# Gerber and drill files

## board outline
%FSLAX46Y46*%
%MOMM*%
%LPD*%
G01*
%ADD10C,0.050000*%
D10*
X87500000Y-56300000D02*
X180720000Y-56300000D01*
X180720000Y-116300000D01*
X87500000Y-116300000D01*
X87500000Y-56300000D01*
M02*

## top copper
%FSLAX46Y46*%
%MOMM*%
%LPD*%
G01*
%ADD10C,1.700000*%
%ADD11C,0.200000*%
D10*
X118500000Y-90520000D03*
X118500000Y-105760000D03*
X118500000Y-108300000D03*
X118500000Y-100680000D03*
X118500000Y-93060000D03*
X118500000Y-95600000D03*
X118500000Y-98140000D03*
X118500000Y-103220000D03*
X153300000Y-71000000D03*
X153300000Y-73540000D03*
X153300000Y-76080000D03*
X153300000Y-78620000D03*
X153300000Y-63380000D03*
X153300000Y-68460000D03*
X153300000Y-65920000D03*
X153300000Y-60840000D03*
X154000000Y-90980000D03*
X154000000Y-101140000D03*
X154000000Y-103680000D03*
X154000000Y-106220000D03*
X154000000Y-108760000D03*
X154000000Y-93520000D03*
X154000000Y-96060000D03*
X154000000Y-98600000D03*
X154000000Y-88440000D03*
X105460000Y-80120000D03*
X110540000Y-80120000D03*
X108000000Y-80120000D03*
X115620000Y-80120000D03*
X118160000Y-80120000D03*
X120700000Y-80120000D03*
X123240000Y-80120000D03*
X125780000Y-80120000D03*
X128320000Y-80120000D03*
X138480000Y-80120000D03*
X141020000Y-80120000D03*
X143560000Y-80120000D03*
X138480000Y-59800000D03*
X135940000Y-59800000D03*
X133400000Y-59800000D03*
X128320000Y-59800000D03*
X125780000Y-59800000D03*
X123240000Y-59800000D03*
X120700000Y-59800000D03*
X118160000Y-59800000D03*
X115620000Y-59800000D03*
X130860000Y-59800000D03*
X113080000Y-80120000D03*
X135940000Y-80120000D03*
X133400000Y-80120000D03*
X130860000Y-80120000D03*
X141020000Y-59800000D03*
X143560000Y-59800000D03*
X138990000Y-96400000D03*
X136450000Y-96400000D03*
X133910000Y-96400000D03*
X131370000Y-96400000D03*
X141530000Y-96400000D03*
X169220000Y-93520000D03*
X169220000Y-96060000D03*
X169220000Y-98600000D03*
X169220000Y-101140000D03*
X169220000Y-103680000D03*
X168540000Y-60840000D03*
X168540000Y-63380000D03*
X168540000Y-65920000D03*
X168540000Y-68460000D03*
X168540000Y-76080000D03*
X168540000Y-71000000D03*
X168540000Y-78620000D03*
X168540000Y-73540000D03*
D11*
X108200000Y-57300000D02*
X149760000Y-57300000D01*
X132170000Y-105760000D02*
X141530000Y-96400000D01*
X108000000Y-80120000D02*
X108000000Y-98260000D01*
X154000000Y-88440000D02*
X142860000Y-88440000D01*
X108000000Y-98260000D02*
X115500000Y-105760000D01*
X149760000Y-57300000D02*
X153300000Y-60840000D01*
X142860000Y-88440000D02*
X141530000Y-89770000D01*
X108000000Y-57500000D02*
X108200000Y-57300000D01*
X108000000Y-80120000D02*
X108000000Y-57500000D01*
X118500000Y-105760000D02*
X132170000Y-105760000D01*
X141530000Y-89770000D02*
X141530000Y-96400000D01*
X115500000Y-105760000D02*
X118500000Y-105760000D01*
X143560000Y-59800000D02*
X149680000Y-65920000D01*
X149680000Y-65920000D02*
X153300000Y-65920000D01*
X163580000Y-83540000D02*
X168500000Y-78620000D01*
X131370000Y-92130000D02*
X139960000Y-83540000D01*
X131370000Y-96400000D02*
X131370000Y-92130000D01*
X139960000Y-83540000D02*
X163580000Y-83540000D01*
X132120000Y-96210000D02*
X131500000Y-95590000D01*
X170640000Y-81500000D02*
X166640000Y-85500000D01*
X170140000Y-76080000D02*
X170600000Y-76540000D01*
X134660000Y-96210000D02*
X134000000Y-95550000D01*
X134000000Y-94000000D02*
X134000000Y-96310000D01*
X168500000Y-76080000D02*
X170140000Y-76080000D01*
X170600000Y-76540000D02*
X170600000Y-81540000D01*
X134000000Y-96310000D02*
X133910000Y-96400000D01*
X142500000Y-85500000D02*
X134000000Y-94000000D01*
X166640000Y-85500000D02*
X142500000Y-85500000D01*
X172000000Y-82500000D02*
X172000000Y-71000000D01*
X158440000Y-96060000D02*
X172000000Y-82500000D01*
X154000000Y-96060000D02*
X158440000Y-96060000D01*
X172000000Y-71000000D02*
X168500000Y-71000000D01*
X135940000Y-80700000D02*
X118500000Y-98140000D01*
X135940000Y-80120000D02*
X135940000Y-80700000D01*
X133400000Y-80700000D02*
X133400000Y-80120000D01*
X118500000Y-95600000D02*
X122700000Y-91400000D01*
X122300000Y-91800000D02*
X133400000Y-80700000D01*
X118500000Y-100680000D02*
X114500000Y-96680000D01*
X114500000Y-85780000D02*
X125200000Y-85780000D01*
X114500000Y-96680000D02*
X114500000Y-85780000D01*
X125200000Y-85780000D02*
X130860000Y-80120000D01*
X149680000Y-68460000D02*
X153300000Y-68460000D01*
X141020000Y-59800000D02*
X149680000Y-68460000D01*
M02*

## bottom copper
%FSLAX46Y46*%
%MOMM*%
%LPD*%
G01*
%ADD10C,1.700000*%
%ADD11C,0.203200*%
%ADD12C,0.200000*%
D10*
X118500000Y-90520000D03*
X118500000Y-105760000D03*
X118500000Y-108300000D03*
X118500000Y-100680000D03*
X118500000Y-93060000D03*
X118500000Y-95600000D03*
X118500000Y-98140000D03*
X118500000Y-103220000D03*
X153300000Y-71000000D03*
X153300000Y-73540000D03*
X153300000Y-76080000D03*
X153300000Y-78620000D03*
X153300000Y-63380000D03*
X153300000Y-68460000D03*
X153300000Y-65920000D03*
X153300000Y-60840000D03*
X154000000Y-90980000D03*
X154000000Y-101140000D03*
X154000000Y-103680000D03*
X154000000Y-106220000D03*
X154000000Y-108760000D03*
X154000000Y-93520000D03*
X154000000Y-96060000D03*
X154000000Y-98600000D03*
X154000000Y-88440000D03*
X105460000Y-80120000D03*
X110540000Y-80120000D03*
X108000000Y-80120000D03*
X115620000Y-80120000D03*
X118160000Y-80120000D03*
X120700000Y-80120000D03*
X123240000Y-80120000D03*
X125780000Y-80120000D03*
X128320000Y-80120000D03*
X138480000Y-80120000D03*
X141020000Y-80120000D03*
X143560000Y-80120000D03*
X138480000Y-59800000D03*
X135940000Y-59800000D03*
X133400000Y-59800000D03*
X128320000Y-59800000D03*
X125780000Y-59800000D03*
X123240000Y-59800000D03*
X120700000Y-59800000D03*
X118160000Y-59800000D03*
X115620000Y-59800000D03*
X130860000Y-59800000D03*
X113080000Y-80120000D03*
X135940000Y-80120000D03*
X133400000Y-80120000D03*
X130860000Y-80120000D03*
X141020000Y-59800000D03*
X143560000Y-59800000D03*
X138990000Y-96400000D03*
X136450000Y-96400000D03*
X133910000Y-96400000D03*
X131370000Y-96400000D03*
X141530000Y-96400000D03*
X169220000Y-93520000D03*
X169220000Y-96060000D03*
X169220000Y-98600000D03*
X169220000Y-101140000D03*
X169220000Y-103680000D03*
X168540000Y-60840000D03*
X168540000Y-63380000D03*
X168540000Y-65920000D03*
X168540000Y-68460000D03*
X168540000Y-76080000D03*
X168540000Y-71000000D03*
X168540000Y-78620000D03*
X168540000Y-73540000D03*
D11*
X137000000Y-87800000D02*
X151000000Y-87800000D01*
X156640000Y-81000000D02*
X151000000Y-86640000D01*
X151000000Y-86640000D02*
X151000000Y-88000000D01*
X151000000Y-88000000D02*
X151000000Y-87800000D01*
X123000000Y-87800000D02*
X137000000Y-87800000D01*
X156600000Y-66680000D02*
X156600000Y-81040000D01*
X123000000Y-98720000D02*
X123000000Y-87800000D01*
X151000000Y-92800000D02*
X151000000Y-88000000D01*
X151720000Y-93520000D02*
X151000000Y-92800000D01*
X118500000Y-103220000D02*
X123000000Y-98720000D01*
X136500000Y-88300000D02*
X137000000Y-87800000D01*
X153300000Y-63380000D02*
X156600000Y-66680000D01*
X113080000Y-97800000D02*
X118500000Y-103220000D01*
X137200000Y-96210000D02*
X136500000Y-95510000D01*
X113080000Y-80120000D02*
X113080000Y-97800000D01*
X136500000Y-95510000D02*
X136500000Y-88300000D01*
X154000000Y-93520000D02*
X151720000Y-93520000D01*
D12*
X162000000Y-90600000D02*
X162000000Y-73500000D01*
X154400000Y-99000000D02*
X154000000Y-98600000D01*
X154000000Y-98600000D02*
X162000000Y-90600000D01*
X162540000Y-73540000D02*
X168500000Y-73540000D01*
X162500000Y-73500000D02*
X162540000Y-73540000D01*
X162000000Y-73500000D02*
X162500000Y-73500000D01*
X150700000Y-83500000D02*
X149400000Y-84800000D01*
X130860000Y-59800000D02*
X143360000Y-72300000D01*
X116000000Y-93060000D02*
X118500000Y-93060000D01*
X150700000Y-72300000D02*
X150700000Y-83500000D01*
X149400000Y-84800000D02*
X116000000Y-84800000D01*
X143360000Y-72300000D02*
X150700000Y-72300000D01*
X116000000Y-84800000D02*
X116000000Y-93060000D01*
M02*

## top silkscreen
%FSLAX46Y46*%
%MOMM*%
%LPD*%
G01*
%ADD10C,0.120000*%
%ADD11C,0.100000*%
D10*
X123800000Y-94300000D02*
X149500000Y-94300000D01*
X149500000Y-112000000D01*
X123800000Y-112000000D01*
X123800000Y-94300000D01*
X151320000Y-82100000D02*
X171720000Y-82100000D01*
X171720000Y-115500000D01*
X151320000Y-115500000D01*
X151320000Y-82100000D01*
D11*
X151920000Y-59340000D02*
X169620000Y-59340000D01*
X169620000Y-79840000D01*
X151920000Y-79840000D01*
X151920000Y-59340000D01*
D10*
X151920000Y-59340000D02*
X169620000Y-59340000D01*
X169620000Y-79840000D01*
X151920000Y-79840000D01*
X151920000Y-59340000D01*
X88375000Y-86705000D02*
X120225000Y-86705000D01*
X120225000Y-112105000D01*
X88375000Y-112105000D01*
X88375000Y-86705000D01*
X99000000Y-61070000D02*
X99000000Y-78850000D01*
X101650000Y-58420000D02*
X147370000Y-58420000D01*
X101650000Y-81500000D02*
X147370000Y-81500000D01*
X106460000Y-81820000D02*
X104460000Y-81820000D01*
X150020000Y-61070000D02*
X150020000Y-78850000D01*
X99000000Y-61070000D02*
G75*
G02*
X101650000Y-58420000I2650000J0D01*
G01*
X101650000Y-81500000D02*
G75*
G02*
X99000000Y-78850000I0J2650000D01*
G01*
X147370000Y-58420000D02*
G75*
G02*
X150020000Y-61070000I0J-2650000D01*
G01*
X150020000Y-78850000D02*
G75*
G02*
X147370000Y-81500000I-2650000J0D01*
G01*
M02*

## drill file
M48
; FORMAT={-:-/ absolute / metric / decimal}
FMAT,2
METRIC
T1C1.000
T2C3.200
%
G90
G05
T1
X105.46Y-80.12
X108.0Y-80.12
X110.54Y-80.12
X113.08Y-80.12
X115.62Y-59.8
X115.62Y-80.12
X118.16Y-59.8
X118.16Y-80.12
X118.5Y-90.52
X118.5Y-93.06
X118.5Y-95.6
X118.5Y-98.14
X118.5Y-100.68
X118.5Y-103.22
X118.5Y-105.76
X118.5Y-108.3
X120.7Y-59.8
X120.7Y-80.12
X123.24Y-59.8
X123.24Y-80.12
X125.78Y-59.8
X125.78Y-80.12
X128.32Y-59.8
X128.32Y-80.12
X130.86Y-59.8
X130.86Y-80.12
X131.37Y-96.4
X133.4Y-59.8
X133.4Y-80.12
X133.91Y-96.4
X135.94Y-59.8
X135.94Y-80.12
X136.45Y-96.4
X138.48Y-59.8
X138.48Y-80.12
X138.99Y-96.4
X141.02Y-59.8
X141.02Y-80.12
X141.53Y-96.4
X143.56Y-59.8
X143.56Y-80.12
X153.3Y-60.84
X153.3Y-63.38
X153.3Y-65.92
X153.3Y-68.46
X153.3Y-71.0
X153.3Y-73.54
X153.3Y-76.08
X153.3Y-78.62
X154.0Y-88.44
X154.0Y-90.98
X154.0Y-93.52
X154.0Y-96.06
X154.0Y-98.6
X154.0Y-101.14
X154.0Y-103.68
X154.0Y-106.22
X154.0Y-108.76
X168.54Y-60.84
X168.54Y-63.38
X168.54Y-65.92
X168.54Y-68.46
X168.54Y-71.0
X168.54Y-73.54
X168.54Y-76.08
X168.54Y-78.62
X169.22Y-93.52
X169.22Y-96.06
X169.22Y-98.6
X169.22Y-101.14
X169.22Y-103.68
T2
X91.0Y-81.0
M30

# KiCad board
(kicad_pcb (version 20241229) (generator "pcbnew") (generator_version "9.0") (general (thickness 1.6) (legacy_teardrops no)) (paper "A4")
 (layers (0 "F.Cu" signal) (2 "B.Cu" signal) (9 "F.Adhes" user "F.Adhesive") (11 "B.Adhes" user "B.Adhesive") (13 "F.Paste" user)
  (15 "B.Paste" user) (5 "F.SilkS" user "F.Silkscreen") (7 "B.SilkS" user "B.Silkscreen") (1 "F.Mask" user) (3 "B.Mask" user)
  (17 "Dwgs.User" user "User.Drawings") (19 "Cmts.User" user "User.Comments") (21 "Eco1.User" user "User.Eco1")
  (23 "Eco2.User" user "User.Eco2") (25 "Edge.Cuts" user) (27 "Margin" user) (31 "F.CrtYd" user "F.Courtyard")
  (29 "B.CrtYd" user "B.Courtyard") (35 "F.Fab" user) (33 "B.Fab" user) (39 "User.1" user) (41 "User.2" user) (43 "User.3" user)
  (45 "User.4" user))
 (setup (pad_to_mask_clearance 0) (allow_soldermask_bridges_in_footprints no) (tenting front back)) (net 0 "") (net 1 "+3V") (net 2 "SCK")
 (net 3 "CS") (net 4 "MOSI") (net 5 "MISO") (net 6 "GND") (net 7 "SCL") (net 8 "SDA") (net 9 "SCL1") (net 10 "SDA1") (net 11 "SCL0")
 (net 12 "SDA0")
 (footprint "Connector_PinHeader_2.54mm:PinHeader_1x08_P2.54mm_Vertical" (layer "F.Cu") (at 118.5 90.52)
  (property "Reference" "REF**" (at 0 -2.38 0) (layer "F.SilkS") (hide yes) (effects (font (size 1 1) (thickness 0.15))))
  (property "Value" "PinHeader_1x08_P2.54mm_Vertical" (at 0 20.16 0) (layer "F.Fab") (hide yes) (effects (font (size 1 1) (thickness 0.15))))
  (pad "1" thru_hole circle (at 0 0) (size 1.7 1.7) (drill 1) (layers "*.Cu" "*.Mask") (remove_unused_layers no))
  (pad "3V" thru_hole circle (at 0 15.24) (size 1.7 1.7) (drill 1) (layers "*.Cu" "*.Mask") (remove_unused_layers no) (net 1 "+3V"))
  (pad "8" thru_hole circle (at 0 17.78) (size 1.7 1.7) (drill 1) (layers "*.Cu" "*.Mask") (remove_unused_layers no))
  (pad "CLK" thru_hole circle (at 0 10.16) (size 1.7 1.7) (drill 1) (layers "*.Cu" "*.Mask") (remove_unused_layers no) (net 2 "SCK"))
  (pad "CS" thru_hole circle (at 0 2.54) (size 1.7 1.7) (drill 1) (layers "*.Cu" "*.Mask") (remove_unused_layers no) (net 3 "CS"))
  (pad "DI" thru_hole circle (at 0 5.08) (size 1.7 1.7) (drill 1) (layers "*.Cu" "*.Mask") (remove_unused_layers no) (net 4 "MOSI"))
  (pad "DO" thru_hole circle (at 0 7.62) (size 1.7 1.7) (drill 1) (layers "*.Cu" "*.Mask") (remove_unused_layers no) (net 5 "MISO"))
  (pad "GND" thru_hole circle (at 0 12.7) (size 1.7 1.7) (drill 1) (layers "*.Cu" "*.Mask") (remove_unused_layers no) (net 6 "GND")))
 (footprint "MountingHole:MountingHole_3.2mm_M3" (layer "F.Cu") (at 91 81)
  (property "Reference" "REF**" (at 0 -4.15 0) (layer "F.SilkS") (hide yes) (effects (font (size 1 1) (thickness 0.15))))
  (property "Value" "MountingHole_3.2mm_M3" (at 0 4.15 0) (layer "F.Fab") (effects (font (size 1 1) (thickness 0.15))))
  (pad "" np_thru_hole circle (at 0 0) (size 3.2 3.2) (drill 3.2) (layers "*.Cu" "*.Mask")))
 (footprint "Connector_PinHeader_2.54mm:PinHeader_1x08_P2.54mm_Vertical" (layer "F.Cu") (at 153.3 60.84)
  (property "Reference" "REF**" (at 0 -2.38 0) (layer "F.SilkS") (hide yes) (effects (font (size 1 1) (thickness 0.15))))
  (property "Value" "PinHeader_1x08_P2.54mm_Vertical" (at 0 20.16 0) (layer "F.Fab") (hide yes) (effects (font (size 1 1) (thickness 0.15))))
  (pad "5" thru_hole circle (at 0 10.16) (size 1.7 1.7) (drill 1) (layers "*.Cu" "*.Mask") (remove_unused_layers no))
  (pad "6" thru_hole circle (at 0 12.7) (size 1.7 1.7) (drill 1) (layers "*.Cu" "*.Mask") (remove_unused_layers no))
  (pad "7" thru_hole circle (at 0 15.24) (size 1.7 1.7) (drill 1) (layers "*.Cu" "*.Mask") (remove_unused_layers no))
  (pad "8" thru_hole circle (at 0 17.78) (size 1.7 1.7) (drill 1) (layers "*.Cu" "*.Mask") (remove_unused_layers no))
  (pad "GND" thru_hole circle (at 0 2.54) (size 1.7 1.7) (drill 1) (layers "*.Cu" "*.Mask") (remove_unused_layers no) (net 6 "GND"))
  (pad "SCL" thru_hole circle (at 0 7.62) (size 1.7 1.7) (drill 1) (layers "*.Cu" "*.Mask") (remove_unused_layers no) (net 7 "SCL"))
  (pad "SDA" thru_hole circle (at 0 5.08) (size 1.7 1.7) (drill 1) (layers "*.Cu" "*.Mask") (remove_unused_layers no) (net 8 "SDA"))
  (pad "VIN" thru_hole circle (at 0 0) (size 1.7 1.7) (drill 1) (layers "*.Cu" "*.Mask") (remove_unused_layers no) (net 1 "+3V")))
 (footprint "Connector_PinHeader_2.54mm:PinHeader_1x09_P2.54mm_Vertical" (layer "F.Cu") (at 154 88.44)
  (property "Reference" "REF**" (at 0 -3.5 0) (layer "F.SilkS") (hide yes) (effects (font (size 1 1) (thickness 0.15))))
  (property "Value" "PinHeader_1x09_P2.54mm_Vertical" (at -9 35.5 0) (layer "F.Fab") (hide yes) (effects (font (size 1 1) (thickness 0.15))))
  (pad "2" thru_hole circle (at 0 2.54) (size 1.7 1.7) (drill 1) (layers "*.Cu" "*.Mask") (remove_unused_layers no))
  (pad "6" thru_hole circle (at 0 12.7) (size 1.7 1.7) (drill 1) (layers "*.Cu" "*.Mask") (remove_unused_layers no))
  (pad "7" thru_hole circle (at 0 15.24) (size 1.7 1.7) (drill 1) (layers "*.Cu" "*.Mask") (remove_unused_layers no))
  (pad "8" thru_hole circle (at 0 17.78) (size 1.7 1.7) (drill 1) (layers "*.Cu" "*.Mask") (remove_unused_layers no))
  (pad "9" thru_hole circle (at 0 20.32) (size 1.7 1.7) (drill 1) (layers "*.Cu" "*.Mask") (remove_unused_layers no))
  (pad "GND" thru_hole circle (at 0 5.08) (size 1.7 1.7) (drill 1) (layers "*.Cu" "*.Mask") (remove_unused_layers no) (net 6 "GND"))
  (pad "SCL" thru_hole circle (at 0 7.62) (size 1.7 1.7) (drill 1) (layers "*.Cu" "*.Mask") (remove_unused_layers no) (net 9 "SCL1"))
  (pad "SDA" thru_hole circle (at 0 10.16) (size 1.7 1.7) (drill 1) (layers "*.Cu" "*.Mask") (remove_unused_layers no) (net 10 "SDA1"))
  (pad "VIN" thru_hole circle (at 0 0) (size 1.7 1.7) (drill 1) (layers "*.Cu" "*.Mask") (remove_unused_layers no) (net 1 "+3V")))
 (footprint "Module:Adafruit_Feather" (layer "F.Cu") (at 105.46 80.12 90)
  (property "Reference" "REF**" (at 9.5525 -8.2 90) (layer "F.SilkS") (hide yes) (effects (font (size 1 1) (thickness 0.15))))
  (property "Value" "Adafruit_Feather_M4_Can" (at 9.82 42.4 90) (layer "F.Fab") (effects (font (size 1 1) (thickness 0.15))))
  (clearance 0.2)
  (fp_line (start 19.05 -6.46) (end 1.27 -6.46) (stroke (width 0.12) (type solid)) (layer "F.SilkS"))
  (fp_line (start 21.7 -3.81) (end 21.7 41.91) (stroke (width 0.12) (type solid)) (layer "F.SilkS"))
  (fp_line (start -1.38 -3.81) (end -1.38 41.91) (stroke (width 0.12) (type solid)) (layer "F.SilkS"))
  (fp_line (start -1.7 1) (end -1.7 -1) (stroke (width 0.12) (type solid)) (layer "F.SilkS"))
  (fp_line (start 19.05 44.56) (end 1.27 44.56) (stroke (width 0.12) (type solid)) (layer "F.SilkS"))
  (fp_arc (start 19.05 -6.46) (mid 20.923833 -5.683833) (end 21.7 -3.81) (stroke (width 0.12) (type solid)) (layer "F.SilkS"))
  (fp_arc (start -1.38 -3.81) (mid -0.603833 -5.683833) (end 1.27 -6.46) (stroke (width 0.12) (type solid)) (layer "F.SilkS"))
  (fp_arc (start 21.7 41.91) (mid 20.923833 43.783833) (end 19.05 44.56) (stroke (width 0.12) (type solid)) (layer "F.SilkS"))
  (fp_arc (start 1.27 44.56) (mid -0.603833 43.783833) (end -1.38 41.91) (stroke (width 0.12) (type solid)) (layer "F.SilkS"))
  (pad "1" thru_hole circle (at 0 0 90) (size 1.7 1.7) (drill 1) (layers "*.Cu" "*.Mask") (remove_unused_layers no))
  (pad "3" thru_hole circle (at 0 5.08 90) (size 1.7 1.7) (drill 1) (layers "*.Cu" "*.Mask") (remove_unused_layers no))
  (pad "3V" thru_hole circle (at 0 2.54 90) (size 1.7 1.7) (drill 1) (layers "*.Cu" "*.Mask") (remove_unused_layers no) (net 1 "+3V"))
  (pad "5" thru_hole circle (at 0 10.16 90) (size 1.7 1.7) (drill 1) (layers "*.Cu" "*.Mask") (remove_unused_layers no))
  (pad "6" thru_hole circle (at 0 12.7 90) (size 1.7 1.7) (drill 1) (layers "*.Cu" "*.Mask") (remove_unused_layers no))
  (pad "7" thru_hole circle (at 0 15.24 90) (size 1.7 1.7) (drill 1) (layers "*.Cu" "*.Mask") (remove_unused_layers no))
  (pad "8" thru_hole circle (at 0 17.78 90) (size 1.7 1.7) (drill 1) (layers "*.Cu" "*.Mask") (remove_unused_layers no))
  (pad "9" thru_hole circle (at 0 20.32 90) (size 1.7 1.7) (drill 1) (layers "*.Cu" "*.Mask") (remove_unused_layers no))
  (pad "10" thru_hole circle (at 0 22.86 90) (size 1.7 1.7) (drill 1) (layers "*.Cu" "*.Mask") (remove_unused_layers no))
  (pad "14" thru_hole circle (at 0 33.02 90) (size 1.7 1.7) (drill 1) (layers "*.Cu" "*.Mask") (remove_unused_layers no))
  (pad "15" thru_hole circle (at 0 35.56 90) (size 1.7 1.7) (drill 1) (layers "*.Cu" "*.Mask") (remove_unused_layers no))
  (pad "16" thru_hole circle (at 0 38.1 90) (size 1.7 1.7) (drill 1) (layers "*.Cu" "*.Mask") (remove_unused_layers no))
  (pad "19" thru_hole circle (at 20.32 33.02 270) (size 1.7 1.7) (drill 1) (layers "*.Cu" "*.Mask") (remove_unused_layers no))
  (pad "20" thru_hole circle (at 20.32 30.48 270) (size 1.7 1.7) (drill 1) (layers "*.Cu" "*.Mask") (remove_unused_layers no))
  (pad "21" thru_hole circle (at 20.32 27.94 270) (size 1.7 1.7) (drill 1) (layers "*.Cu" "*.Mask") (remove_unused_layers no))
  (pad "23" thru_hole circle (at 20.32 22.86 270) (size 1.7 1.7) (drill 1) (layers "*.Cu" "*.Mask") (remove_unused_layers no))
  (pad "24" thru_hole circle (at 20.32 20.32 270) (size 1.7 1.7) (drill 1) (layers "*.Cu" "*.Mask") (remove_unused_layers no))
  (pad "25" thru_hole circle (at 20.32 17.78 270) (size 1.7 1.7) (drill 1) (layers "*.Cu" "*.Mask") (remove_unused_layers no))
  (pad "26" thru_hole circle (at 20.32 15.24 270) (size 1.7 1.7) (drill 1) (layers "*.Cu" "*.Mask") (remove_unused_layers no))
  (pad "27" thru_hole circle (at 20.32 12.7 270) (size 1.7 1.7) (drill 1) (layers "*.Cu" "*.Mask") (remove_unused_layers no))
  (pad "28" thru_hole circle (at 20.32 10.16 270) (size 1.7 1.7) (drill 1) (layers "*.Cu" "*.Mask") (remove_unused_layers no))
  (pad "D10" thru_hole circle (at 20.32 25.4 270) (size 1.7 1.7) (drill 1) (layers "*.Cu" "*.Mask") (remove_unused_layers no) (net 3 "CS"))
  (pad "GND" thru_hole circle (at 0 7.62 90) (size 1.7 1.7) (drill 1) (layers "*.Cu" "*.Mask") (remove_unused_layers no) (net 6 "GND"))
  (pad "MIS" thru_hole circle (at 0 30.48 90) (size 1.7 1.7) (drill 1) (layers "*.Cu" "*.Mask") (remove_unused_layers no) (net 5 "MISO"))
  (pad "MOSI" thru_hole circle (at 0 27.94 90) (size 1.7 1.7) (drill 1) (layers "*.Cu" "*.Mask") (remove_unused_layers no) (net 4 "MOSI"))
  (pad "SCK" thru_hole circle (at 0 25.4 90) (size 1.7 1.7) (drill 1) (layers "*.Cu" "*.Mask") (remove_unused_layers no) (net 2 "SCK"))
  (pad "SCL" thru_hole circle (at 20.32 35.56 270) (size 1.7 1.7) (drill 1) (layers "*.Cu" "*.Mask") (remove_unused_layers no) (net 7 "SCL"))
  (pad "SDA" thru_hole circle (at 20.32 38.1 270) (size 1.7 1.7) (drill 1) (layers "*.Cu" "*.Mask") (remove_unused_layers no) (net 8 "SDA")))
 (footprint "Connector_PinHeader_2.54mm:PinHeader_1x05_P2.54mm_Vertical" (layer "F.Cu") (at 131.37 96.4 90)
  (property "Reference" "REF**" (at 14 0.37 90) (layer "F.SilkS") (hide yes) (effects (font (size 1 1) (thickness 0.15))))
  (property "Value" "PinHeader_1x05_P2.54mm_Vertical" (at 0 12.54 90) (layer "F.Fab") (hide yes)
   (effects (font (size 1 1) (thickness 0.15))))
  (pad "4" thru_hole circle (at 0 7.62 90) (size 1.7 1.7) (drill 1) (layers "*.Cu" "*.Mask") (remove_unused_layers no))
  (pad "GND" thru_hole circle (at 0 5.08 90) (size 1.7 1.7) (drill 1) (layers "*.Cu" "*.Mask") (remove_unused_layers no) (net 6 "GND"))
  (pad "SCL" thru_hole circle (at 0 2.54 90) (size 1.7 1.7) (drill 1) (layers "*.Cu" "*.Mask") (remove_unused_layers no) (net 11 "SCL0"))
  (pad "SDA" thru_hole circle (at 0 0 90) (size 1.7 1.7) (drill 1) (layers "*.Cu" "*.Mask") (remove_unused_layers no) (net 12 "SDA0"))
  (pad "VIN" thru_hole circle (at 0 10.16 90) (size 1.7 1.7) (drill 1) (layers "*.Cu" "*.Mask") (remove_unused_layers no) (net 1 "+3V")))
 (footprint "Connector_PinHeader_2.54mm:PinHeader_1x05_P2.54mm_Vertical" (layer "F.Cu") (at 169.22 93.52)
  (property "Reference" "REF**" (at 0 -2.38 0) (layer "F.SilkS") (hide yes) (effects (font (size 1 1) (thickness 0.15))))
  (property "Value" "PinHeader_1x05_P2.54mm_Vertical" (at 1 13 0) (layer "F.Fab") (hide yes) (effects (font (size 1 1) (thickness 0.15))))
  (pad "1" thru_hole circle (at 0 0) (size 1.7 1.7) (drill 1) (layers "*.Cu" "*.Mask") (remove_unused_layers no))
  (pad "2" thru_hole circle (at 0 2.54) (size 1.7 1.7) (drill 1) (layers "*.Cu" "*.Mask") (remove_unused_layers no))
  (pad "3" thru_hole circle (at 0 5.08) (size 1.7 1.7) (drill 1) (layers "*.Cu" "*.Mask") (remove_unused_layers no))
  (pad "4" thru_hole circle (at 0 7.62) (size 1.7 1.7) (drill 1) (layers "*.Cu" "*.Mask") (remove_unused_layers no))
  (pad "5" thru_hole circle (at 0 10.16) (size 1.7 1.7) (drill 1) (layers "*.Cu" "*.Mask") (remove_unused_layers no)))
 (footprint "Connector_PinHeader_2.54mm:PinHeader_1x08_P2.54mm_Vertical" (layer "F.Cu") (at 168.54 60.84)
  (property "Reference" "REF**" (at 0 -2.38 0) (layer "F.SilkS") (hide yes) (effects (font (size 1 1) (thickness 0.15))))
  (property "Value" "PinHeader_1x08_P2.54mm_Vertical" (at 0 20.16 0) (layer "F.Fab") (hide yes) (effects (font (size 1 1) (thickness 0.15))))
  (pad "1" thru_hole circle (at 0 0) (size 1.7 1.7) (drill 1) (layers "*.Cu" "*.Mask") (remove_unused_layers no))
  (pad "2" thru_hole circle (at 0 2.54) (size 1.7 1.7) (drill 1) (layers "*.Cu" "*.Mask") (remove_unused_layers no))
  (pad "3" thru_hole circle (at 0 5.08) (size 1.7 1.7) (drill 1) (layers "*.Cu" "*.Mask") (remove_unused_layers no))
  (pad "4" thru_hole circle (at 0 7.62) (size 1.7 1.7) (drill 1) (layers "*.Cu" "*.Mask") (remove_unused_layers no))
  (pad "SC0" thru_hole circle (at 0 15.24) (size 1.7 1.7) (drill 1) (layers "*.Cu" "*.Mask") (remove_unused_layers no) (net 11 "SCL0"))
  (pad "SC1" thru_hole circle (at 0 10.16) (size 1.7 1.7) (drill 1) (layers "*.Cu" "*.Mask") (remove_unused_layers no) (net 9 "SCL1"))
  (pad "SD0" thru_hole circle (at 0 17.78) (size 1.7 1.7) (drill 1) (layers "*.Cu" "*.Mask") (remove_unused_layers no) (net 12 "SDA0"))
  (pad "SD1" thru_hole circle (at 0 12.7) (size 1.7 1.7) (drill 1) (layers "*.Cu" "*.Mask") (remove_unused_layers no) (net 10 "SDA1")))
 (gr_rect (start 123.8 94.3) (end 149.5 112) (stroke (width 0.12) (type solid)) (fill no) (layer "F.SilkS"))
 (gr_rect (start 151.32 82.1) (end 171.72 115.5) (stroke (width 0.12) (type solid)) (fill no) (layer "F.SilkS"))
 (gr_rect (start 151.92 59.34) (end 169.62 79.84) (stroke (width 0.1) (type solid)) (fill no) (layer "F.SilkS"))
 (gr_rect (start 151.92 59.34) (end 169.62 79.84) (stroke (width 0.12) (type solid)) (fill no) (layer "F.SilkS"))
 (gr_rect (start 88.375 86.705) (end 120.225 112.105) (stroke (width 0.12) (type solid)) (fill no) (layer "F.SilkS"))
 (gr_rect (start 87.5 56.3) (end 180.72 116.3) (stroke (width 0.05) (type solid)) (fill no) (layer "Edge.Cuts"))
 (segment (start 108.2 57.3) (end 149.76 57.3) (width 0.2) (layer "F.Cu") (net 1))
 (segment (start 132.17 105.76) (end 141.53 96.4) (width 0.2) (layer "F.Cu") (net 1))
 (segment (start 108 80.12) (end 108 98.26) (width 0.2) (layer "F.Cu") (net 1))
 (segment (start 154 88.44) (end 142.86 88.44) (width 0.2) (layer "F.Cu") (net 1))
 (segment (start 108 98.26) (end 115.5 105.76) (width 0.2) (layer "F.Cu") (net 1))
 (segment (start 149.76 57.3) (end 153.3 60.84) (width 0.2) (layer "F.Cu") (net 1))
 (segment (start 142.86 88.44) (end 141.53 89.77) (width 0.2) (layer "F.Cu") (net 1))
 (segment (start 108 57.5) (end 108.2 57.3) (width 0.2) (layer "F.Cu") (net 1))
 (segment (start 108 80.12) (end 108 57.5) (width 0.2) (layer "F.Cu") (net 1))
 (segment (start 118.5 105.76) (end 132.17 105.76) (width 0.2) (layer "F.Cu") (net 1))
 (segment (start 141.53 89.77) (end 141.53 96.4) (width 0.2) (layer "F.Cu") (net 1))
 (segment (start 115.5 105.76) (end 118.5 105.76) (width 0.2) (layer "F.Cu") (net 1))
 (segment (start 137 87.8) (end 151 87.8) (width 0.2032) (layer "B.Cu") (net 6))
 (segment (start 156.64 81) (end 151 86.64) (width 0.2032) (layer "B.Cu") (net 6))
 (segment (start 151 86.64) (end 151 88) (width 0.2032) (layer "B.Cu") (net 6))
 (segment (start 151 88) (end 151 87.8) (width 0.2032) (layer "B.Cu") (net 6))
 (segment (start 123 87.8) (end 137 87.8) (width 0.2032) (layer "B.Cu") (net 6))
 (segment (start 156.6 66.68) (end 156.6 81.04) (width 0.2032) (layer "B.Cu") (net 6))
 (segment (start 123 98.72) (end 123 87.8) (width 0.2032) (layer "B.Cu") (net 6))
 (segment (start 151 92.8) (end 151 88) (width 0.2032) (layer "B.Cu") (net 6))
 (segment (start 151.72 93.52) (end 151 92.8) (width 0.2032) (layer "B.Cu") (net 6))
 (segment (start 118.5 103.22) (end 123 98.72) (width 0.2032) (layer "B.Cu") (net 6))
 (segment (start 136.5 88.3) (end 137 87.8) (width 0.2032) (layer "B.Cu") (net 6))
 (segment (start 153.3 63.38) (end 156.6 66.68) (width 0.2032) (layer "B.Cu") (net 6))
 (segment (start 113.08 97.8) (end 118.5 103.22) (width 0.2032) (layer "B.Cu") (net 6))
 (segment (start 137.2 96.21) (end 136.5 95.51) (width 0.2032) (layer "B.Cu") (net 6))
 (segment (start 113.08 80.12) (end 113.08 97.8) (width 0.2032) (layer "B.Cu") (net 6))
 (segment (start 136.5 95.51) (end 136.5 88.3) (width 0.2032) (layer "B.Cu") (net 6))
 (segment (start 154 93.52) (end 151.72 93.52) (width 0.2032) (layer "B.Cu") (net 6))
 (segment (start 143.56 59.8) (end 149.68 65.92) (width 0.2) (layer "F.Cu") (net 8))
 (segment (start 149.68 65.92) (end 153.3 65.92) (width 0.2) (layer "F.Cu") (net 8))
 (segment (start 163.58 83.54) (end 168.5 78.62) (width 0.2) (layer "F.Cu") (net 12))
 (segment (start 131.37 92.13) (end 139.96 83.54) (width 0.2) (layer "F.Cu") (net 12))
 (segment (start 131.37 96.4) (end 131.37 92.13) (width 0.2) (layer "F.Cu") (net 12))
 (segment (start 139.96 83.54) (end 163.58 83.54) (width 0.2) (layer "F.Cu") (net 12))
 (segment (start 132.12 96.21) (end 131.5 95.59) (width 0.2) (layer "F.Cu") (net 12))
 (segment (start 170.64 81.5) (end 166.64 85.5) (width 0.2) (layer "F.Cu") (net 11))
 (segment (start 170.14 76.08) (end 170.6 76.54) (width 0.2) (layer "F.Cu") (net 11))
 (segment (start 134.66 96.21) (end 134 95.55) (width 0.2) (layer "F.Cu") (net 11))
 (segment (start 134 94) (end 134 96.31) (width 0.2) (layer "F.Cu") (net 11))
 (segment (start 168.5 76.08) (end 170.14 76.08) (width 0.2) (layer "F.Cu") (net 11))
 (segment (start 170.6 76.54) (end 170.6 81.54) (width 0.2) (layer "F.Cu") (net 11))
 (segment (start 134 96.31) (end 133.91 96.4) (width 0.2) (layer "F.Cu") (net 11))
 (segment (start 142.5 85.5) (end 134 94) (width 0.2) (layer "F.Cu") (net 11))
 (segment (start 166.64 85.5) (end 142.5 85.5) (width 0.2) (layer "F.Cu") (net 11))
 (segment (start 162 90.6) (end 162 73.5) (width 0.2) (layer "B.Cu") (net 10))
 (segment (start 154.4 99) (end 154 98.6) (width 0.2) (layer "B.Cu") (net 10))
 (segment (start 154 98.6) (end 162 90.6) (width 0.2) (layer "B.Cu") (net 10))
 (segment (start 162.54 73.54) (end 168.5 73.54) (width 0.2) (layer "B.Cu") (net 10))
 (segment (start 162.5 73.5) (end 162.54 73.54) (width 0.2) (layer "B.Cu") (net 10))
 (segment (start 162 73.5) (end 162.5 73.5) (width 0.2) (layer "B.Cu") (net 10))
 (segment (start 172 82.5) (end 172 71) (width 0.2) (layer "F.Cu") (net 9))
 (segment (start 158.44 96.06) (end 172 82.5) (width 0.2) (layer "F.Cu") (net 9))
 (segment (start 154 96.06) (end 158.44 96.06) (width 0.2) (layer "F.Cu") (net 9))
 (segment (start 172 71) (end 168.5 71) (width 0.2) (layer "F.Cu") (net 9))
 (segment (start 135.94 80.7) (end 118.5 98.14) (width 0.2) (layer "F.Cu") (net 5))
 (segment (start 135.94 80.12) (end 135.94 80.7) (width 0.2) (layer "F.Cu") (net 5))
 (segment (start 133.4 80.7) (end 133.4 80.12) (width 0.2) (layer "F.Cu") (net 4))
 (segment (start 118.5 95.6) (end 122.7 91.4) (width 0.2) (layer "F.Cu") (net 4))
 (segment (start 122.3 91.8) (end 133.4 80.7) (width 0.2) (layer "F.Cu") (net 4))
 (segment (start 118.5 100.68) (end 114.5 96.68) (width 0.2) (layer "F.Cu") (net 2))
 (segment (start 114.5 85.78) (end 125.2 85.78) (width 0.2) (layer "F.Cu") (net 2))
 (segment (start 114.5 96.68) (end 114.5 85.78) (width 0.2) (layer "F.Cu") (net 2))
 (segment (start 125.2 85.78) (end 130.86 80.12) (width 0.2) (layer "F.Cu") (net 2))
 (segment (start 149.68 68.46) (end 153.3 68.46) (width 0.2) (layer "F.Cu") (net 7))
 (segment (start 141.02 59.8) (end 149.68 68.46) (width 0.2) (layer "F.Cu") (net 7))
 (segment (start 150.7 83.5) (end 149.4 84.8) (width 0.2) (layer "B.Cu") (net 3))
 (segment (start 130.86 59.8) (end 143.36 72.3) (width 0.2) (layer "B.Cu") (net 3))
 (segment (start 116 93.06) (end 118.5 93.06) (width 0.2) (layer "B.Cu") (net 3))
 (segment (start 150.7 72.3) (end 150.7 83.5) (width 0.2) (layer "B.Cu") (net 3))
 (segment (start 149.4 84.8) (end 116 84.8) (width 0.2) (layer "B.Cu") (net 3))
 (segment (start 143.36 72.3) (end 150.7 72.3) (width 0.2) (layer "B.Cu") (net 3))
 (segment (start 116 84.8) (end 116 93.06) (width 0.2) (layer "B.Cu") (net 3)))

